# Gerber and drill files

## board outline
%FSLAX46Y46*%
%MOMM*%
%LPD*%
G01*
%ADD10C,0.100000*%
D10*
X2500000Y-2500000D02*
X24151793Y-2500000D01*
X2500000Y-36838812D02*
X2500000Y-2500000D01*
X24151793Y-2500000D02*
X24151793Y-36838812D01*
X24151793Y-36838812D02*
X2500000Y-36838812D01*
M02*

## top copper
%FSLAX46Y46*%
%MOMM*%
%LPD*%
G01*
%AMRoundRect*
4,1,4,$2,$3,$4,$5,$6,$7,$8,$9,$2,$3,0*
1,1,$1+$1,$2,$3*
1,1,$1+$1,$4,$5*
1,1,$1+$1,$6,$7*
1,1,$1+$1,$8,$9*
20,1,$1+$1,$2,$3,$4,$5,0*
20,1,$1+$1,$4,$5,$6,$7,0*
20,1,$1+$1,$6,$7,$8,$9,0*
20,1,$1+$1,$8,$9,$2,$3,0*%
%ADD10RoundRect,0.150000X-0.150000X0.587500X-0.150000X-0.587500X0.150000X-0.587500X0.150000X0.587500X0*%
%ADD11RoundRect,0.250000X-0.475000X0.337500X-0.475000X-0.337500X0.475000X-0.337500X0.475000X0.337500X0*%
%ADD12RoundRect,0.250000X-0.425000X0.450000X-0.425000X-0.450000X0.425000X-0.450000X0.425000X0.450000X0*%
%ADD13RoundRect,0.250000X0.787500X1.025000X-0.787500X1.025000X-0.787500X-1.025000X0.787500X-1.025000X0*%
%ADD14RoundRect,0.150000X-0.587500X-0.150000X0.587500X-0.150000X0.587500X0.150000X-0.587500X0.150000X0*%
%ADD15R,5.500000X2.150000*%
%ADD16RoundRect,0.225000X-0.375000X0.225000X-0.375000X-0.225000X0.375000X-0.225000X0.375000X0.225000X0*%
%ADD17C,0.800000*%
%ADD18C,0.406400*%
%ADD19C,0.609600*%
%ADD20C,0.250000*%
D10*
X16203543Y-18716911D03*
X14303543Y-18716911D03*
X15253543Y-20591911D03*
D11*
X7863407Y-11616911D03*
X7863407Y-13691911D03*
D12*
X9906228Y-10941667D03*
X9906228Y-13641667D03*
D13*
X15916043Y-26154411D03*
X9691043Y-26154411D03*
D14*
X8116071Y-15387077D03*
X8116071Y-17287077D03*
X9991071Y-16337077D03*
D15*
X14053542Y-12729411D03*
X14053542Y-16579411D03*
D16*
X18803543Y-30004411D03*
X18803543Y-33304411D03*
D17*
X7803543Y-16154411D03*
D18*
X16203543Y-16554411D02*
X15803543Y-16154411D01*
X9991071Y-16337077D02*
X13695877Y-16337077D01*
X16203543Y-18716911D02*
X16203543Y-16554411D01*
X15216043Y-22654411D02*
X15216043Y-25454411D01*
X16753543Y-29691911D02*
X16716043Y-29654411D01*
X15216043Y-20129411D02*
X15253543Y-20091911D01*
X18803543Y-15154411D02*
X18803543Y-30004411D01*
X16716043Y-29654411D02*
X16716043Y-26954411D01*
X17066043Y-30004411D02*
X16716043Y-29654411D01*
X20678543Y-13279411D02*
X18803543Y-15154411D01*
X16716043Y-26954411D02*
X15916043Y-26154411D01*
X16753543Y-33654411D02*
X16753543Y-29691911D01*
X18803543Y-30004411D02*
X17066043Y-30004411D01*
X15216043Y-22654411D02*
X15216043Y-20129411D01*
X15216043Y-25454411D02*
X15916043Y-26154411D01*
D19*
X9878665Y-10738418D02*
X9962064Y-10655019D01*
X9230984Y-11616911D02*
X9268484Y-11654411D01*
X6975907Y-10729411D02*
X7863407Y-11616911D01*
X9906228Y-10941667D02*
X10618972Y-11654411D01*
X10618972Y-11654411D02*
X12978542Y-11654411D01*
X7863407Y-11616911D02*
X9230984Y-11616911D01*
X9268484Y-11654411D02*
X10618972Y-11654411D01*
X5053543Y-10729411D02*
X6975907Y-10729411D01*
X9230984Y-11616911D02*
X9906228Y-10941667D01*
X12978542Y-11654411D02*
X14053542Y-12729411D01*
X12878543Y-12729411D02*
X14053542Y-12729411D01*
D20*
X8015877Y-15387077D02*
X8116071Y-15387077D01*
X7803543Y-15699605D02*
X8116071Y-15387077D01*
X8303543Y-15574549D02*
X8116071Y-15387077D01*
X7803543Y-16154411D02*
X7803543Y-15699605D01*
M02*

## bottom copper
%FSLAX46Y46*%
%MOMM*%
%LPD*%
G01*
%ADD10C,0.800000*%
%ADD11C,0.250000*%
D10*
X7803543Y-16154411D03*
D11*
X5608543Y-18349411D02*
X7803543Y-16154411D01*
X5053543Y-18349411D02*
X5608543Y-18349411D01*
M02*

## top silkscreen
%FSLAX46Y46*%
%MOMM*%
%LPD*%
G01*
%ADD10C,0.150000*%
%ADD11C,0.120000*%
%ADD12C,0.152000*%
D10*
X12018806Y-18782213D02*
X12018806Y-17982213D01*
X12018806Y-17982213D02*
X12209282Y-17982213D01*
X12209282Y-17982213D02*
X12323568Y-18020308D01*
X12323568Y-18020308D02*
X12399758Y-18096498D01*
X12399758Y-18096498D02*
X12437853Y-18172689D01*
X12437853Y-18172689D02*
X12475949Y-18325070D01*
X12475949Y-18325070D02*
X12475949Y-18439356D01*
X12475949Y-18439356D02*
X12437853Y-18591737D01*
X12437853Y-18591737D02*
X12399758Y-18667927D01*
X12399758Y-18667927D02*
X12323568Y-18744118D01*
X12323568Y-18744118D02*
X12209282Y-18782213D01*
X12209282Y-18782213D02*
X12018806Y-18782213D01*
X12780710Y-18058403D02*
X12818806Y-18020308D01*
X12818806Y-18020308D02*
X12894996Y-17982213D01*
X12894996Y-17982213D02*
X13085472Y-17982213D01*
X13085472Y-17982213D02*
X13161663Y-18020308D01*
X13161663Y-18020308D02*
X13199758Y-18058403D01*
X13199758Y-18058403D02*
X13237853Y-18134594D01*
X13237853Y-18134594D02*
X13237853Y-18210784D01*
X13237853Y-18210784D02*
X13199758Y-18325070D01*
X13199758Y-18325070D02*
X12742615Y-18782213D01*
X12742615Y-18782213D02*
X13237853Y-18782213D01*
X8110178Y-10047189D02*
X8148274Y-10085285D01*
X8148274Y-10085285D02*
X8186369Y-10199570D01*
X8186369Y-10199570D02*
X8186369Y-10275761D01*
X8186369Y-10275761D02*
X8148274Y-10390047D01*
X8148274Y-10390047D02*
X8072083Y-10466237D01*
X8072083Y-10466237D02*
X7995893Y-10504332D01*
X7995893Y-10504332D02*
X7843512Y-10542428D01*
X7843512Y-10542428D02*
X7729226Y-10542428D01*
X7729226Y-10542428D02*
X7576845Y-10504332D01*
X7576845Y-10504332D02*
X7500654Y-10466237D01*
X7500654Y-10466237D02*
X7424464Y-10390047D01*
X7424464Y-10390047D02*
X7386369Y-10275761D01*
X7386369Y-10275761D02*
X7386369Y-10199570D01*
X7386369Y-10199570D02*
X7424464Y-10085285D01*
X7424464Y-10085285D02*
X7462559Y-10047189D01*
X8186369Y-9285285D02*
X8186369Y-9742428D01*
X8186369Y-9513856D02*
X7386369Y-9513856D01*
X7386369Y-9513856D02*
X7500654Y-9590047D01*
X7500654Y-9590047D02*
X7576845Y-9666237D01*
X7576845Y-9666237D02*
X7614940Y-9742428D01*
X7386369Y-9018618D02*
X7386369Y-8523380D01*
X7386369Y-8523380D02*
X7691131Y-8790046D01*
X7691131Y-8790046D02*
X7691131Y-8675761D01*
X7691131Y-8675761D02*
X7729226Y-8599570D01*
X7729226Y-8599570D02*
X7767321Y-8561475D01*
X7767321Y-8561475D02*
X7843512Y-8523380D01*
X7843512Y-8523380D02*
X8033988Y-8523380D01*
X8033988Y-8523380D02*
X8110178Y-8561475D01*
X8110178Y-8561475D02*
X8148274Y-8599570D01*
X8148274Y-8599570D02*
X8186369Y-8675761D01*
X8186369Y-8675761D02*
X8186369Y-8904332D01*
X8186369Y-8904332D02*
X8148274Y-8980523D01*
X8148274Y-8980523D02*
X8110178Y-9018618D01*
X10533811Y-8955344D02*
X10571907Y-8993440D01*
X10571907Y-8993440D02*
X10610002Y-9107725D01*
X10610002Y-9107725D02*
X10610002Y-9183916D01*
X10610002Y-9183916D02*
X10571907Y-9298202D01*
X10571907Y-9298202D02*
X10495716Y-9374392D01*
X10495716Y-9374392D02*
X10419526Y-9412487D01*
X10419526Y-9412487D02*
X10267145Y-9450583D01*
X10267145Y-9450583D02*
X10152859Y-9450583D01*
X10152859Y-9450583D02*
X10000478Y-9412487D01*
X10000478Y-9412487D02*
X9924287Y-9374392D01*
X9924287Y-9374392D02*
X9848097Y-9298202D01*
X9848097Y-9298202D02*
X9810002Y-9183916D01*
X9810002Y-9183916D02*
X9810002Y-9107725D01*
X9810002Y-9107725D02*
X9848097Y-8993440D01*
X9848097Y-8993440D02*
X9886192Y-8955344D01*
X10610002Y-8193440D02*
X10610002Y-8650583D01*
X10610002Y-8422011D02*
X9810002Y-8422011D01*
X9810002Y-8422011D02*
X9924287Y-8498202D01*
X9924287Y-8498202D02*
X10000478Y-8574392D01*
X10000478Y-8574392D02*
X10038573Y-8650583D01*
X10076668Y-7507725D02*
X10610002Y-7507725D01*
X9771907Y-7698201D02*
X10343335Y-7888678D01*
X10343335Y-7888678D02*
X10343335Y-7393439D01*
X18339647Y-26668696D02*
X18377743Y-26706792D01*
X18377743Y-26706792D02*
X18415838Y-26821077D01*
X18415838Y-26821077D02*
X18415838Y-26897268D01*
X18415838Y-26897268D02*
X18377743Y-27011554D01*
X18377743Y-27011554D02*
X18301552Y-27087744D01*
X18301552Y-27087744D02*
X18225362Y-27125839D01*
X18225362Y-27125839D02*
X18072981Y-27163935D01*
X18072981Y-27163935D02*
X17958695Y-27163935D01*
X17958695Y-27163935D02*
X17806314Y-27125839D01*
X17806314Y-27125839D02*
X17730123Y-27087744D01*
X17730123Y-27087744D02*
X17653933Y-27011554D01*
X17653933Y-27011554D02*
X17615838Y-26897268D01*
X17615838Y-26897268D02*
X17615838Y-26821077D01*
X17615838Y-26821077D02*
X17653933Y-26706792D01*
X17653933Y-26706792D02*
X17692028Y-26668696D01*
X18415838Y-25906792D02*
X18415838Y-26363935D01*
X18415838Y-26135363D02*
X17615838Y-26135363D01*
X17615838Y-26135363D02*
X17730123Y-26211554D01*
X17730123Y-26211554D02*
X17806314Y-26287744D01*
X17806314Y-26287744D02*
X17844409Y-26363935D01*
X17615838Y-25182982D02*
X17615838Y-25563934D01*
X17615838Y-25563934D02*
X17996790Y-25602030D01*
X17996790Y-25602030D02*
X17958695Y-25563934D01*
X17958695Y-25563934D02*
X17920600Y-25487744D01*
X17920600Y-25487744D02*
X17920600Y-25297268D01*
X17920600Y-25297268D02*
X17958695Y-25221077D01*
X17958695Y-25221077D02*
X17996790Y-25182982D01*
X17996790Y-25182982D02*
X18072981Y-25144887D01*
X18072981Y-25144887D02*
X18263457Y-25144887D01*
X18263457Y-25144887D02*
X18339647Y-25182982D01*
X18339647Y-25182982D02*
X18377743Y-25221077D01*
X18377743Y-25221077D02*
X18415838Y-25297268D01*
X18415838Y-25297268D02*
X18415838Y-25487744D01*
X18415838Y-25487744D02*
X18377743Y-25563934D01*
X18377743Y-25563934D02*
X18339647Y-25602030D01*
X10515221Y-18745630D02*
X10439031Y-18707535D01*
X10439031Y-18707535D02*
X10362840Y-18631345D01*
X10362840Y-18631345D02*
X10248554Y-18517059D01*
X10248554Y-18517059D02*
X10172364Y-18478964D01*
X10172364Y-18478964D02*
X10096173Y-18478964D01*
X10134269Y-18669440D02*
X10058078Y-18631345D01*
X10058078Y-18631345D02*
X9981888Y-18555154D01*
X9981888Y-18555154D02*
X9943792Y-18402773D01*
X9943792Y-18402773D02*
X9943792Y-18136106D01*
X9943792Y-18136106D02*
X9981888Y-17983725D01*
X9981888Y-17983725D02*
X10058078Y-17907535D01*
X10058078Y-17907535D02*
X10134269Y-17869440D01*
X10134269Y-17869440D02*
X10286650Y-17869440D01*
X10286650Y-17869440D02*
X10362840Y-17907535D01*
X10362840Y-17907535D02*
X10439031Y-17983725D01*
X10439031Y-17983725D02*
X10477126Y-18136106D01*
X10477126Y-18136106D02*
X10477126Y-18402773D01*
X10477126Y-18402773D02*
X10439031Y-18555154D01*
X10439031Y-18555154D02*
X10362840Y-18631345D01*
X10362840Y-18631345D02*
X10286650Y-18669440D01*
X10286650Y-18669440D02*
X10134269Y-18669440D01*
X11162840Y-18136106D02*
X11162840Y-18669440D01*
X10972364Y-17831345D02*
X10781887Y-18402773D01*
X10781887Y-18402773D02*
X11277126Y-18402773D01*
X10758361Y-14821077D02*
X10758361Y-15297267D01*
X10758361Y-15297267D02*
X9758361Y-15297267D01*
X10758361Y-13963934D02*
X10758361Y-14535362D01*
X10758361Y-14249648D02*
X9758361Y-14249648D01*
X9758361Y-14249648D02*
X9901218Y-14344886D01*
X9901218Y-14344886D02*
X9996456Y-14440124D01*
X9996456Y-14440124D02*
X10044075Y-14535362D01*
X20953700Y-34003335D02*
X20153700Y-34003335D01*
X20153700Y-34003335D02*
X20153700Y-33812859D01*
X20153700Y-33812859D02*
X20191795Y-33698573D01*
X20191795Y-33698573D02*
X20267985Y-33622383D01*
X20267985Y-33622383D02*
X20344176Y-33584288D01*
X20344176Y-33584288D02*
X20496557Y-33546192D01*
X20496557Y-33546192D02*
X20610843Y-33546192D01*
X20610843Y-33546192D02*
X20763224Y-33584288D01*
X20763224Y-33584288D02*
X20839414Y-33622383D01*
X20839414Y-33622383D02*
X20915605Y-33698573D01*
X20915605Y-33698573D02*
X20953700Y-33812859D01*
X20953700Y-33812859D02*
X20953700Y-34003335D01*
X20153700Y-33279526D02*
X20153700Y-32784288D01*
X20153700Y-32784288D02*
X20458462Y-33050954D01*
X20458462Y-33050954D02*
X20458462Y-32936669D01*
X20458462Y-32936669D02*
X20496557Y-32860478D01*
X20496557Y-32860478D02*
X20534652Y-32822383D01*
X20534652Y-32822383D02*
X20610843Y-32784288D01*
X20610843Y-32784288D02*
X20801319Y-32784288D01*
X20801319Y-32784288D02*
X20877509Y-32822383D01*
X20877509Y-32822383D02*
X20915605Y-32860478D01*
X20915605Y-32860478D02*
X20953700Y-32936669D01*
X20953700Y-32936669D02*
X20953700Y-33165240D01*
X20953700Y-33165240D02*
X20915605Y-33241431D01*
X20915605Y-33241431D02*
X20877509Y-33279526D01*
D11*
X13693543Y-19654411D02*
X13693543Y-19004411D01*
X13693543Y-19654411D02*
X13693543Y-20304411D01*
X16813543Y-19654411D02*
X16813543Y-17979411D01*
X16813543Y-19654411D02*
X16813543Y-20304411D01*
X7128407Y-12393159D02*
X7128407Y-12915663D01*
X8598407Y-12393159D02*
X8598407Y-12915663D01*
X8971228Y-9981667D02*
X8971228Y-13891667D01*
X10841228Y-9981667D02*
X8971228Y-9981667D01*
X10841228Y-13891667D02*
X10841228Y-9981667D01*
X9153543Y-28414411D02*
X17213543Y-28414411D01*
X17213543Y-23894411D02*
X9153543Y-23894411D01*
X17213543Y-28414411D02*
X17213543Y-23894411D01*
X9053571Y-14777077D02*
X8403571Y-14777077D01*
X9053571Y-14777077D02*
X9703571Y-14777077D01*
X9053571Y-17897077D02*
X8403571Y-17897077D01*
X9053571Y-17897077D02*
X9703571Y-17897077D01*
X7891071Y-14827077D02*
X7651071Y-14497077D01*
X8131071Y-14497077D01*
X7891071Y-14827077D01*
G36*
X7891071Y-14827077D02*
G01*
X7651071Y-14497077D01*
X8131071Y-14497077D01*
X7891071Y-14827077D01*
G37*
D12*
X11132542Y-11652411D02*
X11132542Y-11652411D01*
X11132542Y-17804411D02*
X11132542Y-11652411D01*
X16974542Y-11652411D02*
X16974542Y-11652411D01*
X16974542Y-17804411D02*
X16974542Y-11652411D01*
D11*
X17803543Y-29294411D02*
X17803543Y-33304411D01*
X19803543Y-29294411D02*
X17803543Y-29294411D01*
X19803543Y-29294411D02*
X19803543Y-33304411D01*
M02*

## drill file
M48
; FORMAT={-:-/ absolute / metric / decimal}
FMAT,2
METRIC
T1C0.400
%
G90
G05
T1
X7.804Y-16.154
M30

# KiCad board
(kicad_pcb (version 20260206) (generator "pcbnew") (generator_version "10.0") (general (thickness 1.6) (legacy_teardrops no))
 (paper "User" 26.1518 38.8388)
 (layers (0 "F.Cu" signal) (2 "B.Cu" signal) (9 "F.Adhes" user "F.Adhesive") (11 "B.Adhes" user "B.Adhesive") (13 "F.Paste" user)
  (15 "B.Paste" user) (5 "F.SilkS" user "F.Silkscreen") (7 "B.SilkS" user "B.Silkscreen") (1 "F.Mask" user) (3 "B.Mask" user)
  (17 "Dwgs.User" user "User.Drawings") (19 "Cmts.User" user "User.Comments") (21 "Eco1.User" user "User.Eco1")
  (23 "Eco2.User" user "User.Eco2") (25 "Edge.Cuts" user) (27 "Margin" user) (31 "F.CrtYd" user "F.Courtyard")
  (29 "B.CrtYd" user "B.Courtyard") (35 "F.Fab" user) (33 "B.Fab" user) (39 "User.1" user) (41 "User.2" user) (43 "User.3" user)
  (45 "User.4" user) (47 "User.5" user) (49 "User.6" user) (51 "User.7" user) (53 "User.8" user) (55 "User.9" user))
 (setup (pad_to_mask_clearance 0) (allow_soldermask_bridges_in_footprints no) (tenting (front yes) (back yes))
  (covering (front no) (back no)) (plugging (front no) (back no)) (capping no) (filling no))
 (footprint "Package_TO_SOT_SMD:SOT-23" (layer "F.Cu") (at 15.253543 19.654411 -90)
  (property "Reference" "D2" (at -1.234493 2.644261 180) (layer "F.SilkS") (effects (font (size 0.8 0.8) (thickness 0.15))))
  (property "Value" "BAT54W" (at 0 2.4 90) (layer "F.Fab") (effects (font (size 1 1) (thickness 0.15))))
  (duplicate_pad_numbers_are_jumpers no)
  (fp_line (start 0 1.56) (end -0.65 1.56) (stroke (width 0.12) (type solid)) (layer "F.SilkS"))
  (fp_line (start 0 1.56) (end 0.65 1.56) (stroke (width 0.12) (type solid)) (layer "F.SilkS"))
  (fp_line (start 0 -1.56) (end -1.675 -1.56) (stroke (width 0.12) (type solid)) (layer "F.SilkS"))
  (fp_line (start 0 -1.56) (end 0.65 -1.56) (stroke (width 0.12) (type solid)) (layer "F.SilkS"))
  (pad "1" smd roundrect (at -0.9375 -0.95 270) (size 1.475 0.6) (layers "F.Cu" "F.Mask" "F.Paste") (roundrect_rratio 0.25)
   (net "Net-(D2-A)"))
  (pad "2" smd roundrect (at -0.9375 0.95 270) (size 1.475 0.6) (layers "F.Cu" "F.Mask" "F.Paste") (roundrect_rratio 0.25)
   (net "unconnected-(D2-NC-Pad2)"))
  (pad "3" smd roundrect (at 0.9375 0 270) (size 1.475 0.6) (layers "F.Cu" "F.Mask" "F.Paste") (roundrect_rratio 0.25) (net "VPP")))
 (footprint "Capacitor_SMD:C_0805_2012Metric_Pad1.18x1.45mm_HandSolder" (layer "F.Cu") (at 7.863407 12.654411 -90)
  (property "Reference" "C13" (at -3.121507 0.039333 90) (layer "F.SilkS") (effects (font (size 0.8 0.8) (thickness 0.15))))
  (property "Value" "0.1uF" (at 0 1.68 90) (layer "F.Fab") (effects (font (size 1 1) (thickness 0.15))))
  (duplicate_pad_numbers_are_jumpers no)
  (fp_line (start -0.261252 0.735) (end 0.261252 0.735) (stroke (width 0.12) (type solid)) (layer "F.SilkS"))
  (fp_line (start -0.261252 -0.735) (end 0.261252 -0.735) (stroke (width 0.12) (type solid)) (layer "F.SilkS"))
  (pad "1" smd roundrect (at -1.0375 0 270) (size 1.175 1.45) (layers "F.Cu" "F.Mask" "F.Paste") (roundrect_rratio 0.2127659574)
   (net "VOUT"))
  (pad "2" smd roundrect (at 1.0375 0 270) (size 1.175 1.45) (layers "F.Cu" "F.Mask" "F.Paste") (roundrect_rratio 0.2127659574) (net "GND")))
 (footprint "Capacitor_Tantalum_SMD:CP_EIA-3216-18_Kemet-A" (layer "F.Cu") (at 9.906228 12.291667 -90)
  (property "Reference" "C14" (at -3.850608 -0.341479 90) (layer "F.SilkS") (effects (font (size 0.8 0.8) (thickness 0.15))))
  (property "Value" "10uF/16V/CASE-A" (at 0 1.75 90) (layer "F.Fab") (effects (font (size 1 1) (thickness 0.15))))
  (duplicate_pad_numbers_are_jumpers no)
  (fp_line (start -2.31 0.935) (end 1.6 0.935) (stroke (width 0.12) (type solid)) (layer "F.SilkS"))
  (fp_line (start -2.31 -0.935) (end -2.31 0.935) (stroke (width 0.12) (type solid)) (layer "F.SilkS"))
  (fp_line (start 1.6 -0.935) (end -2.31 -0.935) (stroke (width 0.12) (type solid)) (layer "F.SilkS"))
  (pad "1" smd roundrect (at -1.35 0 270) (size 1.4 1.35) (layers "F.Cu" "F.Mask" "F.Paste") (roundrect_rratio 0.1851851852) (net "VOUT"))
  (pad "2" smd roundrect (at 1.35 0 270) (size 1.4 1.35) (layers "F.Cu" "F.Mask" "F.Paste") (roundrect_rratio 0.1851851852) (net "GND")))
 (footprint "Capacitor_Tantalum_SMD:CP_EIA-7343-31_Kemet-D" (layer "F.Cu") (at 12.803543 26.154411 180)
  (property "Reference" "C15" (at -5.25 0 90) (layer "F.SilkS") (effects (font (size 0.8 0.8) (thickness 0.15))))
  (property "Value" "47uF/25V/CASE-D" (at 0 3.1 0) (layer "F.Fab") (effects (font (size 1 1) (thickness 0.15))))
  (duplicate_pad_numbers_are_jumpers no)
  (fp_line (start 3.65 -2.26) (end -4.41 -2.26) (stroke (width 0.12) (type solid)) (layer "F.SilkS"))
  (fp_line (start -4.41 2.26) (end 3.65 2.26) (stroke (width 0.12) (type solid)) (layer "F.SilkS"))
  (fp_line (start -4.41 -2.26) (end -4.41 2.26) (stroke (width 0.12) (type solid)) (layer "F.SilkS"))
  (pad "1" smd roundrect (at -3.1125 0 180) (size 2.075 2.55) (layers "F.Cu" "F.Mask" "F.Paste") (roundrect_rratio 0.1204819277) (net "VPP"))
  (pad "2" smd roundrect (at 3.1125 0 180) (size 2.075 2.55) (layers "F.Cu" "F.Mask" "F.Paste") (roundrect_rratio 0.1204819277) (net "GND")))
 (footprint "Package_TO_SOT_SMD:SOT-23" (layer "F.Cu") (at 9.053571 16.337077)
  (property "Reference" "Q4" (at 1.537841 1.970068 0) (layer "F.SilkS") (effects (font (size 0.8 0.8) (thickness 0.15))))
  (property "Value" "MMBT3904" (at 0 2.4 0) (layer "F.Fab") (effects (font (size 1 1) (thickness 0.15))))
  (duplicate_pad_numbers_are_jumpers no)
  (fp_line (start 0 -1.56) (end -0.65 -1.56) (stroke (width 0.12) (type solid)) (layer "F.SilkS"))
  (fp_line (start 0 -1.56) (end 0.65 -1.56) (stroke (width 0.12) (type solid)) (layer "F.SilkS"))
  (fp_line (start 0 1.56) (end -0.65 1.56) (stroke (width 0.12) (type solid)) (layer "F.SilkS"))
  (fp_line (start 0 1.56) (end 0.65 1.56) (stroke (width 0.12) (type solid)) (layer "F.SilkS"))
  (fp_poly
   (pts (xy -1.1625 -1.51) (xy -1.4025 -1.84) (xy -0.9225 -1.84) (xy -1.1625 -1.51)) (stroke (width 0.12) (type solid)) (fill yes)
   (layer "F.SilkS"))
  (pad "1" smd roundrect (at -0.9375 -0.95) (size 1.475 0.6) (layers "F.Cu" "F.Mask" "F.Paste") (roundrect_rratio 0.25) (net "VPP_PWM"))
  (pad "2" smd roundrect (at -0.9375 0.95) (size 1.475 0.6) (layers "F.Cu" "F.Mask" "F.Paste") (roundrect_rratio 0.25) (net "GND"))
  (pad "3" smd roundrect (at 0.9375 0) (size 1.475 0.6) (layers "F.Cu" "F.Mask" "F.Paste") (roundrect_rratio 0.25) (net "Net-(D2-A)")))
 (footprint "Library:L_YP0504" (layer "F.Cu") (at 14.053542 14.654411 90)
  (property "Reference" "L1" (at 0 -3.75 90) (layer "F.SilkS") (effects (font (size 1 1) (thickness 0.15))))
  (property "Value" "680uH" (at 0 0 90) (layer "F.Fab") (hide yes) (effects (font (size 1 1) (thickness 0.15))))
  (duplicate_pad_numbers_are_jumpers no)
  (fp_line (start 3.002 -2.921) (end 3.002 -2.921) (stroke (width 0.152) (type solid)) (layer "F.SilkS"))
  (fp_line (start -3.15 -2.921) (end 3.002 -2.921) (stroke (width 0.152) (type solid)) (layer "F.SilkS"))
  (fp_line (start 3.002 2.921) (end 3.002 2.921) (stroke (width 0.152) (type solid)) (layer "F.SilkS"))
  (fp_line (start -3.15 2.921) (end 3.002 2.921) (stroke (width 0.152) (type solid)) (layer "F.SilkS"))
  (pad "1" smd rect (at 1.925 0 90) (size 2.15 5.5) (layers "F.Cu" "F.Mask" "F.Paste") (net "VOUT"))
  (pad "2" smd rect (at -1.925 0 90) (size 2.15 5.5) (layers "F.Cu" "F.Mask" "F.Paste") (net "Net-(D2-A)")))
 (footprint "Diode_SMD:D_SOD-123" (layer "F.Cu") (at 18.803543 31.654411 -90)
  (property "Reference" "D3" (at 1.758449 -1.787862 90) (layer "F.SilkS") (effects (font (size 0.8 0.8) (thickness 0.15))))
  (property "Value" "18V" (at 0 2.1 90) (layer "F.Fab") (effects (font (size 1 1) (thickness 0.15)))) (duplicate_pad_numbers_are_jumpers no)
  (fp_line (start -2.36 1) (end 1.65 1) (stroke (width 0.12) (type solid)) (layer "F.SilkS"))
  (fp_line (start -2.36 -1) (end -2.36 1) (stroke (width 0.12) (type solid)) (layer "F.SilkS"))
  (fp_line (start -2.36 -1) (end 1.65 -1) (stroke (width 0.12) (type solid)) (layer "F.SilkS"))
  (pad "1" smd roundrect (at -1.65 0 270) (size 0.9 1.2) (layers "F.Cu" "F.Mask" "F.Paste") (roundrect_rratio 0.25) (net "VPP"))
  (pad "2" smd roundrect (at 1.65 0 270) (size 0.9 1.2) (layers "F.Cu" "F.Mask" "F.Paste") (roundrect_rratio 0.25) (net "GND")))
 (gr_line (start 2.5 2.5) (end 24.151793 2.5) (stroke (width 0.1) (type default)) (layer "Edge.Cuts"))
 (gr_line (start 2.5 36.838812) (end 2.5 2.5) (stroke (width 0.1) (type default)) (layer "Edge.Cuts"))
 (gr_line (start 24.151793 2.5) (end 24.151793 36.838812) (stroke (width 0.1) (type default)) (layer "Edge.Cuts"))
 (gr_line (start 24.151793 36.838812) (end 2.5 36.838812) (stroke (width 0.1) (type default)) (layer "Edge.Cuts"))
 (segment (start 16.203543 16.554411) (end 15.803543 16.154411) (width 0.4064) (layer "F.Cu") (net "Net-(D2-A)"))
 (segment (start 9.991071 16.337077) (end 13.695877 16.337077) (width 0.4064) (layer "F.Cu") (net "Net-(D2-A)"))
 (segment (start 16.203543 18.716911) (end 16.203543 16.554411) (width 0.4064) (layer "F.Cu") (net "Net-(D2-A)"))
 (segment (start 15.216043 22.654411) (end 15.216043 25.454411) (width 0.4064) (layer "F.Cu") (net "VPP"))
 (segment (start 16.753543 29.691911) (end 16.716043 29.654411) (width 0.4064) (layer "F.Cu") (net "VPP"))
 (segment (start 15.216043 20.129411) (end 15.253543 20.091911) (width 0.4064) (layer "F.Cu") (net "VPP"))
 (segment (start 18.803543 15.154411) (end 18.803543 30.004411) (width 0.4064) (layer "F.Cu") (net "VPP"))
 (segment (start 16.716043 29.654411) (end 16.716043 26.954411) (width 0.4064) (layer "F.Cu") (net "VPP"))
 (segment (start 17.066043 30.004411) (end 16.716043 29.654411) (width 0.4064) (layer "F.Cu") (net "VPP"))
 (segment (start 20.678543 13.279411) (end 18.803543 15.154411) (width 0.4064) (layer "F.Cu") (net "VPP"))
 (segment (start 16.716043 26.954411) (end 15.916043 26.154411) (width 0.4064) (layer "F.Cu") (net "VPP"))
 (segment (start 16.753543 33.654411) (end 16.753543 29.691911) (width 0.4064) (layer "F.Cu") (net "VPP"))
 (segment (start 18.803543 30.004411) (end 17.066043 30.004411) (width 0.4064) (layer "F.Cu") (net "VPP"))
 (segment (start 15.216043 22.654411) (end 15.216043 20.129411) (width 0.4064) (layer "F.Cu") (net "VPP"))
 (segment (start 15.216043 25.454411) (end 15.916043 26.154411) (width 0.4064) (layer "F.Cu") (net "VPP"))
 (segment (start 9.878665 10.738418) (end 9.962064 10.655019) (width 0.6096) (layer "F.Cu") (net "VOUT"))
 (segment (start 9.230984 11.616911) (end 9.268484 11.654411) (width 0.6096) (layer "F.Cu") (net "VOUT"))
 (segment (start 6.975907 10.729411) (end 7.863407 11.616911) (width 0.6096) (layer "F.Cu") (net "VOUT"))
 (segment (start 9.906228 10.941667) (end 10.618972 11.654411) (width 0.6096) (layer "F.Cu") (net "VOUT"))
 (segment (start 10.618972 11.654411) (end 12.978542 11.654411) (width 0.6096) (layer "F.Cu") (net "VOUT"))
 (segment (start 7.863407 11.616911) (end 9.230984 11.616911) (width 0.6096) (layer "F.Cu") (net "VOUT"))
 (segment (start 9.268484 11.654411) (end 10.618972 11.654411) (width 0.6096) (layer "F.Cu") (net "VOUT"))
 (segment (start 5.053543 10.729411) (end 6.975907 10.729411) (width 0.6096) (layer "F.Cu") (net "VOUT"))
 (segment (start 9.230984 11.616911) (end 9.906228 10.941667) (width 0.6096) (layer "F.Cu") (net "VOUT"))
 (segment (start 12.978542 11.654411) (end 14.053542 12.729411) (width 0.6096) (layer "F.Cu") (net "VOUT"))
 (segment (start 12.878543 12.729411) (end 14.053542 12.729411) (width 0.6096) (layer "F.Cu") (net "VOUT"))
 (segment (start 8.015877 15.387077) (end 8.116071 15.387077) (width 0.25) (layer "F.Cu") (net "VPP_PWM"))
 (segment (start 7.803543 15.699605) (end 8.116071 15.387077) (width 0.25) (layer "F.Cu") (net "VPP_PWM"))
 (segment (start 8.303543 15.574549) (end 8.116071 15.387077) (width 0.25) (layer "F.Cu") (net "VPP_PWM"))
 (segment (start 7.803543 16.154411) (end 7.803543 15.699605) (width 0.25) (layer "F.Cu") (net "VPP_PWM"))
 (via (at 7.803543 16.154411) (size 0.8) (drill 0.4) (layers "F.Cu" "B.Cu") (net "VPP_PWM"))
 (segment (start 5.608543 18.349411) (end 7.803543 16.154411) (width 0.25) (layer "B.Cu") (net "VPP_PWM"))
 (segment (start 5.053543 18.349411) (end 5.608543 18.349411) (width 0.25) (layer "B.Cu") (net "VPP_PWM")))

